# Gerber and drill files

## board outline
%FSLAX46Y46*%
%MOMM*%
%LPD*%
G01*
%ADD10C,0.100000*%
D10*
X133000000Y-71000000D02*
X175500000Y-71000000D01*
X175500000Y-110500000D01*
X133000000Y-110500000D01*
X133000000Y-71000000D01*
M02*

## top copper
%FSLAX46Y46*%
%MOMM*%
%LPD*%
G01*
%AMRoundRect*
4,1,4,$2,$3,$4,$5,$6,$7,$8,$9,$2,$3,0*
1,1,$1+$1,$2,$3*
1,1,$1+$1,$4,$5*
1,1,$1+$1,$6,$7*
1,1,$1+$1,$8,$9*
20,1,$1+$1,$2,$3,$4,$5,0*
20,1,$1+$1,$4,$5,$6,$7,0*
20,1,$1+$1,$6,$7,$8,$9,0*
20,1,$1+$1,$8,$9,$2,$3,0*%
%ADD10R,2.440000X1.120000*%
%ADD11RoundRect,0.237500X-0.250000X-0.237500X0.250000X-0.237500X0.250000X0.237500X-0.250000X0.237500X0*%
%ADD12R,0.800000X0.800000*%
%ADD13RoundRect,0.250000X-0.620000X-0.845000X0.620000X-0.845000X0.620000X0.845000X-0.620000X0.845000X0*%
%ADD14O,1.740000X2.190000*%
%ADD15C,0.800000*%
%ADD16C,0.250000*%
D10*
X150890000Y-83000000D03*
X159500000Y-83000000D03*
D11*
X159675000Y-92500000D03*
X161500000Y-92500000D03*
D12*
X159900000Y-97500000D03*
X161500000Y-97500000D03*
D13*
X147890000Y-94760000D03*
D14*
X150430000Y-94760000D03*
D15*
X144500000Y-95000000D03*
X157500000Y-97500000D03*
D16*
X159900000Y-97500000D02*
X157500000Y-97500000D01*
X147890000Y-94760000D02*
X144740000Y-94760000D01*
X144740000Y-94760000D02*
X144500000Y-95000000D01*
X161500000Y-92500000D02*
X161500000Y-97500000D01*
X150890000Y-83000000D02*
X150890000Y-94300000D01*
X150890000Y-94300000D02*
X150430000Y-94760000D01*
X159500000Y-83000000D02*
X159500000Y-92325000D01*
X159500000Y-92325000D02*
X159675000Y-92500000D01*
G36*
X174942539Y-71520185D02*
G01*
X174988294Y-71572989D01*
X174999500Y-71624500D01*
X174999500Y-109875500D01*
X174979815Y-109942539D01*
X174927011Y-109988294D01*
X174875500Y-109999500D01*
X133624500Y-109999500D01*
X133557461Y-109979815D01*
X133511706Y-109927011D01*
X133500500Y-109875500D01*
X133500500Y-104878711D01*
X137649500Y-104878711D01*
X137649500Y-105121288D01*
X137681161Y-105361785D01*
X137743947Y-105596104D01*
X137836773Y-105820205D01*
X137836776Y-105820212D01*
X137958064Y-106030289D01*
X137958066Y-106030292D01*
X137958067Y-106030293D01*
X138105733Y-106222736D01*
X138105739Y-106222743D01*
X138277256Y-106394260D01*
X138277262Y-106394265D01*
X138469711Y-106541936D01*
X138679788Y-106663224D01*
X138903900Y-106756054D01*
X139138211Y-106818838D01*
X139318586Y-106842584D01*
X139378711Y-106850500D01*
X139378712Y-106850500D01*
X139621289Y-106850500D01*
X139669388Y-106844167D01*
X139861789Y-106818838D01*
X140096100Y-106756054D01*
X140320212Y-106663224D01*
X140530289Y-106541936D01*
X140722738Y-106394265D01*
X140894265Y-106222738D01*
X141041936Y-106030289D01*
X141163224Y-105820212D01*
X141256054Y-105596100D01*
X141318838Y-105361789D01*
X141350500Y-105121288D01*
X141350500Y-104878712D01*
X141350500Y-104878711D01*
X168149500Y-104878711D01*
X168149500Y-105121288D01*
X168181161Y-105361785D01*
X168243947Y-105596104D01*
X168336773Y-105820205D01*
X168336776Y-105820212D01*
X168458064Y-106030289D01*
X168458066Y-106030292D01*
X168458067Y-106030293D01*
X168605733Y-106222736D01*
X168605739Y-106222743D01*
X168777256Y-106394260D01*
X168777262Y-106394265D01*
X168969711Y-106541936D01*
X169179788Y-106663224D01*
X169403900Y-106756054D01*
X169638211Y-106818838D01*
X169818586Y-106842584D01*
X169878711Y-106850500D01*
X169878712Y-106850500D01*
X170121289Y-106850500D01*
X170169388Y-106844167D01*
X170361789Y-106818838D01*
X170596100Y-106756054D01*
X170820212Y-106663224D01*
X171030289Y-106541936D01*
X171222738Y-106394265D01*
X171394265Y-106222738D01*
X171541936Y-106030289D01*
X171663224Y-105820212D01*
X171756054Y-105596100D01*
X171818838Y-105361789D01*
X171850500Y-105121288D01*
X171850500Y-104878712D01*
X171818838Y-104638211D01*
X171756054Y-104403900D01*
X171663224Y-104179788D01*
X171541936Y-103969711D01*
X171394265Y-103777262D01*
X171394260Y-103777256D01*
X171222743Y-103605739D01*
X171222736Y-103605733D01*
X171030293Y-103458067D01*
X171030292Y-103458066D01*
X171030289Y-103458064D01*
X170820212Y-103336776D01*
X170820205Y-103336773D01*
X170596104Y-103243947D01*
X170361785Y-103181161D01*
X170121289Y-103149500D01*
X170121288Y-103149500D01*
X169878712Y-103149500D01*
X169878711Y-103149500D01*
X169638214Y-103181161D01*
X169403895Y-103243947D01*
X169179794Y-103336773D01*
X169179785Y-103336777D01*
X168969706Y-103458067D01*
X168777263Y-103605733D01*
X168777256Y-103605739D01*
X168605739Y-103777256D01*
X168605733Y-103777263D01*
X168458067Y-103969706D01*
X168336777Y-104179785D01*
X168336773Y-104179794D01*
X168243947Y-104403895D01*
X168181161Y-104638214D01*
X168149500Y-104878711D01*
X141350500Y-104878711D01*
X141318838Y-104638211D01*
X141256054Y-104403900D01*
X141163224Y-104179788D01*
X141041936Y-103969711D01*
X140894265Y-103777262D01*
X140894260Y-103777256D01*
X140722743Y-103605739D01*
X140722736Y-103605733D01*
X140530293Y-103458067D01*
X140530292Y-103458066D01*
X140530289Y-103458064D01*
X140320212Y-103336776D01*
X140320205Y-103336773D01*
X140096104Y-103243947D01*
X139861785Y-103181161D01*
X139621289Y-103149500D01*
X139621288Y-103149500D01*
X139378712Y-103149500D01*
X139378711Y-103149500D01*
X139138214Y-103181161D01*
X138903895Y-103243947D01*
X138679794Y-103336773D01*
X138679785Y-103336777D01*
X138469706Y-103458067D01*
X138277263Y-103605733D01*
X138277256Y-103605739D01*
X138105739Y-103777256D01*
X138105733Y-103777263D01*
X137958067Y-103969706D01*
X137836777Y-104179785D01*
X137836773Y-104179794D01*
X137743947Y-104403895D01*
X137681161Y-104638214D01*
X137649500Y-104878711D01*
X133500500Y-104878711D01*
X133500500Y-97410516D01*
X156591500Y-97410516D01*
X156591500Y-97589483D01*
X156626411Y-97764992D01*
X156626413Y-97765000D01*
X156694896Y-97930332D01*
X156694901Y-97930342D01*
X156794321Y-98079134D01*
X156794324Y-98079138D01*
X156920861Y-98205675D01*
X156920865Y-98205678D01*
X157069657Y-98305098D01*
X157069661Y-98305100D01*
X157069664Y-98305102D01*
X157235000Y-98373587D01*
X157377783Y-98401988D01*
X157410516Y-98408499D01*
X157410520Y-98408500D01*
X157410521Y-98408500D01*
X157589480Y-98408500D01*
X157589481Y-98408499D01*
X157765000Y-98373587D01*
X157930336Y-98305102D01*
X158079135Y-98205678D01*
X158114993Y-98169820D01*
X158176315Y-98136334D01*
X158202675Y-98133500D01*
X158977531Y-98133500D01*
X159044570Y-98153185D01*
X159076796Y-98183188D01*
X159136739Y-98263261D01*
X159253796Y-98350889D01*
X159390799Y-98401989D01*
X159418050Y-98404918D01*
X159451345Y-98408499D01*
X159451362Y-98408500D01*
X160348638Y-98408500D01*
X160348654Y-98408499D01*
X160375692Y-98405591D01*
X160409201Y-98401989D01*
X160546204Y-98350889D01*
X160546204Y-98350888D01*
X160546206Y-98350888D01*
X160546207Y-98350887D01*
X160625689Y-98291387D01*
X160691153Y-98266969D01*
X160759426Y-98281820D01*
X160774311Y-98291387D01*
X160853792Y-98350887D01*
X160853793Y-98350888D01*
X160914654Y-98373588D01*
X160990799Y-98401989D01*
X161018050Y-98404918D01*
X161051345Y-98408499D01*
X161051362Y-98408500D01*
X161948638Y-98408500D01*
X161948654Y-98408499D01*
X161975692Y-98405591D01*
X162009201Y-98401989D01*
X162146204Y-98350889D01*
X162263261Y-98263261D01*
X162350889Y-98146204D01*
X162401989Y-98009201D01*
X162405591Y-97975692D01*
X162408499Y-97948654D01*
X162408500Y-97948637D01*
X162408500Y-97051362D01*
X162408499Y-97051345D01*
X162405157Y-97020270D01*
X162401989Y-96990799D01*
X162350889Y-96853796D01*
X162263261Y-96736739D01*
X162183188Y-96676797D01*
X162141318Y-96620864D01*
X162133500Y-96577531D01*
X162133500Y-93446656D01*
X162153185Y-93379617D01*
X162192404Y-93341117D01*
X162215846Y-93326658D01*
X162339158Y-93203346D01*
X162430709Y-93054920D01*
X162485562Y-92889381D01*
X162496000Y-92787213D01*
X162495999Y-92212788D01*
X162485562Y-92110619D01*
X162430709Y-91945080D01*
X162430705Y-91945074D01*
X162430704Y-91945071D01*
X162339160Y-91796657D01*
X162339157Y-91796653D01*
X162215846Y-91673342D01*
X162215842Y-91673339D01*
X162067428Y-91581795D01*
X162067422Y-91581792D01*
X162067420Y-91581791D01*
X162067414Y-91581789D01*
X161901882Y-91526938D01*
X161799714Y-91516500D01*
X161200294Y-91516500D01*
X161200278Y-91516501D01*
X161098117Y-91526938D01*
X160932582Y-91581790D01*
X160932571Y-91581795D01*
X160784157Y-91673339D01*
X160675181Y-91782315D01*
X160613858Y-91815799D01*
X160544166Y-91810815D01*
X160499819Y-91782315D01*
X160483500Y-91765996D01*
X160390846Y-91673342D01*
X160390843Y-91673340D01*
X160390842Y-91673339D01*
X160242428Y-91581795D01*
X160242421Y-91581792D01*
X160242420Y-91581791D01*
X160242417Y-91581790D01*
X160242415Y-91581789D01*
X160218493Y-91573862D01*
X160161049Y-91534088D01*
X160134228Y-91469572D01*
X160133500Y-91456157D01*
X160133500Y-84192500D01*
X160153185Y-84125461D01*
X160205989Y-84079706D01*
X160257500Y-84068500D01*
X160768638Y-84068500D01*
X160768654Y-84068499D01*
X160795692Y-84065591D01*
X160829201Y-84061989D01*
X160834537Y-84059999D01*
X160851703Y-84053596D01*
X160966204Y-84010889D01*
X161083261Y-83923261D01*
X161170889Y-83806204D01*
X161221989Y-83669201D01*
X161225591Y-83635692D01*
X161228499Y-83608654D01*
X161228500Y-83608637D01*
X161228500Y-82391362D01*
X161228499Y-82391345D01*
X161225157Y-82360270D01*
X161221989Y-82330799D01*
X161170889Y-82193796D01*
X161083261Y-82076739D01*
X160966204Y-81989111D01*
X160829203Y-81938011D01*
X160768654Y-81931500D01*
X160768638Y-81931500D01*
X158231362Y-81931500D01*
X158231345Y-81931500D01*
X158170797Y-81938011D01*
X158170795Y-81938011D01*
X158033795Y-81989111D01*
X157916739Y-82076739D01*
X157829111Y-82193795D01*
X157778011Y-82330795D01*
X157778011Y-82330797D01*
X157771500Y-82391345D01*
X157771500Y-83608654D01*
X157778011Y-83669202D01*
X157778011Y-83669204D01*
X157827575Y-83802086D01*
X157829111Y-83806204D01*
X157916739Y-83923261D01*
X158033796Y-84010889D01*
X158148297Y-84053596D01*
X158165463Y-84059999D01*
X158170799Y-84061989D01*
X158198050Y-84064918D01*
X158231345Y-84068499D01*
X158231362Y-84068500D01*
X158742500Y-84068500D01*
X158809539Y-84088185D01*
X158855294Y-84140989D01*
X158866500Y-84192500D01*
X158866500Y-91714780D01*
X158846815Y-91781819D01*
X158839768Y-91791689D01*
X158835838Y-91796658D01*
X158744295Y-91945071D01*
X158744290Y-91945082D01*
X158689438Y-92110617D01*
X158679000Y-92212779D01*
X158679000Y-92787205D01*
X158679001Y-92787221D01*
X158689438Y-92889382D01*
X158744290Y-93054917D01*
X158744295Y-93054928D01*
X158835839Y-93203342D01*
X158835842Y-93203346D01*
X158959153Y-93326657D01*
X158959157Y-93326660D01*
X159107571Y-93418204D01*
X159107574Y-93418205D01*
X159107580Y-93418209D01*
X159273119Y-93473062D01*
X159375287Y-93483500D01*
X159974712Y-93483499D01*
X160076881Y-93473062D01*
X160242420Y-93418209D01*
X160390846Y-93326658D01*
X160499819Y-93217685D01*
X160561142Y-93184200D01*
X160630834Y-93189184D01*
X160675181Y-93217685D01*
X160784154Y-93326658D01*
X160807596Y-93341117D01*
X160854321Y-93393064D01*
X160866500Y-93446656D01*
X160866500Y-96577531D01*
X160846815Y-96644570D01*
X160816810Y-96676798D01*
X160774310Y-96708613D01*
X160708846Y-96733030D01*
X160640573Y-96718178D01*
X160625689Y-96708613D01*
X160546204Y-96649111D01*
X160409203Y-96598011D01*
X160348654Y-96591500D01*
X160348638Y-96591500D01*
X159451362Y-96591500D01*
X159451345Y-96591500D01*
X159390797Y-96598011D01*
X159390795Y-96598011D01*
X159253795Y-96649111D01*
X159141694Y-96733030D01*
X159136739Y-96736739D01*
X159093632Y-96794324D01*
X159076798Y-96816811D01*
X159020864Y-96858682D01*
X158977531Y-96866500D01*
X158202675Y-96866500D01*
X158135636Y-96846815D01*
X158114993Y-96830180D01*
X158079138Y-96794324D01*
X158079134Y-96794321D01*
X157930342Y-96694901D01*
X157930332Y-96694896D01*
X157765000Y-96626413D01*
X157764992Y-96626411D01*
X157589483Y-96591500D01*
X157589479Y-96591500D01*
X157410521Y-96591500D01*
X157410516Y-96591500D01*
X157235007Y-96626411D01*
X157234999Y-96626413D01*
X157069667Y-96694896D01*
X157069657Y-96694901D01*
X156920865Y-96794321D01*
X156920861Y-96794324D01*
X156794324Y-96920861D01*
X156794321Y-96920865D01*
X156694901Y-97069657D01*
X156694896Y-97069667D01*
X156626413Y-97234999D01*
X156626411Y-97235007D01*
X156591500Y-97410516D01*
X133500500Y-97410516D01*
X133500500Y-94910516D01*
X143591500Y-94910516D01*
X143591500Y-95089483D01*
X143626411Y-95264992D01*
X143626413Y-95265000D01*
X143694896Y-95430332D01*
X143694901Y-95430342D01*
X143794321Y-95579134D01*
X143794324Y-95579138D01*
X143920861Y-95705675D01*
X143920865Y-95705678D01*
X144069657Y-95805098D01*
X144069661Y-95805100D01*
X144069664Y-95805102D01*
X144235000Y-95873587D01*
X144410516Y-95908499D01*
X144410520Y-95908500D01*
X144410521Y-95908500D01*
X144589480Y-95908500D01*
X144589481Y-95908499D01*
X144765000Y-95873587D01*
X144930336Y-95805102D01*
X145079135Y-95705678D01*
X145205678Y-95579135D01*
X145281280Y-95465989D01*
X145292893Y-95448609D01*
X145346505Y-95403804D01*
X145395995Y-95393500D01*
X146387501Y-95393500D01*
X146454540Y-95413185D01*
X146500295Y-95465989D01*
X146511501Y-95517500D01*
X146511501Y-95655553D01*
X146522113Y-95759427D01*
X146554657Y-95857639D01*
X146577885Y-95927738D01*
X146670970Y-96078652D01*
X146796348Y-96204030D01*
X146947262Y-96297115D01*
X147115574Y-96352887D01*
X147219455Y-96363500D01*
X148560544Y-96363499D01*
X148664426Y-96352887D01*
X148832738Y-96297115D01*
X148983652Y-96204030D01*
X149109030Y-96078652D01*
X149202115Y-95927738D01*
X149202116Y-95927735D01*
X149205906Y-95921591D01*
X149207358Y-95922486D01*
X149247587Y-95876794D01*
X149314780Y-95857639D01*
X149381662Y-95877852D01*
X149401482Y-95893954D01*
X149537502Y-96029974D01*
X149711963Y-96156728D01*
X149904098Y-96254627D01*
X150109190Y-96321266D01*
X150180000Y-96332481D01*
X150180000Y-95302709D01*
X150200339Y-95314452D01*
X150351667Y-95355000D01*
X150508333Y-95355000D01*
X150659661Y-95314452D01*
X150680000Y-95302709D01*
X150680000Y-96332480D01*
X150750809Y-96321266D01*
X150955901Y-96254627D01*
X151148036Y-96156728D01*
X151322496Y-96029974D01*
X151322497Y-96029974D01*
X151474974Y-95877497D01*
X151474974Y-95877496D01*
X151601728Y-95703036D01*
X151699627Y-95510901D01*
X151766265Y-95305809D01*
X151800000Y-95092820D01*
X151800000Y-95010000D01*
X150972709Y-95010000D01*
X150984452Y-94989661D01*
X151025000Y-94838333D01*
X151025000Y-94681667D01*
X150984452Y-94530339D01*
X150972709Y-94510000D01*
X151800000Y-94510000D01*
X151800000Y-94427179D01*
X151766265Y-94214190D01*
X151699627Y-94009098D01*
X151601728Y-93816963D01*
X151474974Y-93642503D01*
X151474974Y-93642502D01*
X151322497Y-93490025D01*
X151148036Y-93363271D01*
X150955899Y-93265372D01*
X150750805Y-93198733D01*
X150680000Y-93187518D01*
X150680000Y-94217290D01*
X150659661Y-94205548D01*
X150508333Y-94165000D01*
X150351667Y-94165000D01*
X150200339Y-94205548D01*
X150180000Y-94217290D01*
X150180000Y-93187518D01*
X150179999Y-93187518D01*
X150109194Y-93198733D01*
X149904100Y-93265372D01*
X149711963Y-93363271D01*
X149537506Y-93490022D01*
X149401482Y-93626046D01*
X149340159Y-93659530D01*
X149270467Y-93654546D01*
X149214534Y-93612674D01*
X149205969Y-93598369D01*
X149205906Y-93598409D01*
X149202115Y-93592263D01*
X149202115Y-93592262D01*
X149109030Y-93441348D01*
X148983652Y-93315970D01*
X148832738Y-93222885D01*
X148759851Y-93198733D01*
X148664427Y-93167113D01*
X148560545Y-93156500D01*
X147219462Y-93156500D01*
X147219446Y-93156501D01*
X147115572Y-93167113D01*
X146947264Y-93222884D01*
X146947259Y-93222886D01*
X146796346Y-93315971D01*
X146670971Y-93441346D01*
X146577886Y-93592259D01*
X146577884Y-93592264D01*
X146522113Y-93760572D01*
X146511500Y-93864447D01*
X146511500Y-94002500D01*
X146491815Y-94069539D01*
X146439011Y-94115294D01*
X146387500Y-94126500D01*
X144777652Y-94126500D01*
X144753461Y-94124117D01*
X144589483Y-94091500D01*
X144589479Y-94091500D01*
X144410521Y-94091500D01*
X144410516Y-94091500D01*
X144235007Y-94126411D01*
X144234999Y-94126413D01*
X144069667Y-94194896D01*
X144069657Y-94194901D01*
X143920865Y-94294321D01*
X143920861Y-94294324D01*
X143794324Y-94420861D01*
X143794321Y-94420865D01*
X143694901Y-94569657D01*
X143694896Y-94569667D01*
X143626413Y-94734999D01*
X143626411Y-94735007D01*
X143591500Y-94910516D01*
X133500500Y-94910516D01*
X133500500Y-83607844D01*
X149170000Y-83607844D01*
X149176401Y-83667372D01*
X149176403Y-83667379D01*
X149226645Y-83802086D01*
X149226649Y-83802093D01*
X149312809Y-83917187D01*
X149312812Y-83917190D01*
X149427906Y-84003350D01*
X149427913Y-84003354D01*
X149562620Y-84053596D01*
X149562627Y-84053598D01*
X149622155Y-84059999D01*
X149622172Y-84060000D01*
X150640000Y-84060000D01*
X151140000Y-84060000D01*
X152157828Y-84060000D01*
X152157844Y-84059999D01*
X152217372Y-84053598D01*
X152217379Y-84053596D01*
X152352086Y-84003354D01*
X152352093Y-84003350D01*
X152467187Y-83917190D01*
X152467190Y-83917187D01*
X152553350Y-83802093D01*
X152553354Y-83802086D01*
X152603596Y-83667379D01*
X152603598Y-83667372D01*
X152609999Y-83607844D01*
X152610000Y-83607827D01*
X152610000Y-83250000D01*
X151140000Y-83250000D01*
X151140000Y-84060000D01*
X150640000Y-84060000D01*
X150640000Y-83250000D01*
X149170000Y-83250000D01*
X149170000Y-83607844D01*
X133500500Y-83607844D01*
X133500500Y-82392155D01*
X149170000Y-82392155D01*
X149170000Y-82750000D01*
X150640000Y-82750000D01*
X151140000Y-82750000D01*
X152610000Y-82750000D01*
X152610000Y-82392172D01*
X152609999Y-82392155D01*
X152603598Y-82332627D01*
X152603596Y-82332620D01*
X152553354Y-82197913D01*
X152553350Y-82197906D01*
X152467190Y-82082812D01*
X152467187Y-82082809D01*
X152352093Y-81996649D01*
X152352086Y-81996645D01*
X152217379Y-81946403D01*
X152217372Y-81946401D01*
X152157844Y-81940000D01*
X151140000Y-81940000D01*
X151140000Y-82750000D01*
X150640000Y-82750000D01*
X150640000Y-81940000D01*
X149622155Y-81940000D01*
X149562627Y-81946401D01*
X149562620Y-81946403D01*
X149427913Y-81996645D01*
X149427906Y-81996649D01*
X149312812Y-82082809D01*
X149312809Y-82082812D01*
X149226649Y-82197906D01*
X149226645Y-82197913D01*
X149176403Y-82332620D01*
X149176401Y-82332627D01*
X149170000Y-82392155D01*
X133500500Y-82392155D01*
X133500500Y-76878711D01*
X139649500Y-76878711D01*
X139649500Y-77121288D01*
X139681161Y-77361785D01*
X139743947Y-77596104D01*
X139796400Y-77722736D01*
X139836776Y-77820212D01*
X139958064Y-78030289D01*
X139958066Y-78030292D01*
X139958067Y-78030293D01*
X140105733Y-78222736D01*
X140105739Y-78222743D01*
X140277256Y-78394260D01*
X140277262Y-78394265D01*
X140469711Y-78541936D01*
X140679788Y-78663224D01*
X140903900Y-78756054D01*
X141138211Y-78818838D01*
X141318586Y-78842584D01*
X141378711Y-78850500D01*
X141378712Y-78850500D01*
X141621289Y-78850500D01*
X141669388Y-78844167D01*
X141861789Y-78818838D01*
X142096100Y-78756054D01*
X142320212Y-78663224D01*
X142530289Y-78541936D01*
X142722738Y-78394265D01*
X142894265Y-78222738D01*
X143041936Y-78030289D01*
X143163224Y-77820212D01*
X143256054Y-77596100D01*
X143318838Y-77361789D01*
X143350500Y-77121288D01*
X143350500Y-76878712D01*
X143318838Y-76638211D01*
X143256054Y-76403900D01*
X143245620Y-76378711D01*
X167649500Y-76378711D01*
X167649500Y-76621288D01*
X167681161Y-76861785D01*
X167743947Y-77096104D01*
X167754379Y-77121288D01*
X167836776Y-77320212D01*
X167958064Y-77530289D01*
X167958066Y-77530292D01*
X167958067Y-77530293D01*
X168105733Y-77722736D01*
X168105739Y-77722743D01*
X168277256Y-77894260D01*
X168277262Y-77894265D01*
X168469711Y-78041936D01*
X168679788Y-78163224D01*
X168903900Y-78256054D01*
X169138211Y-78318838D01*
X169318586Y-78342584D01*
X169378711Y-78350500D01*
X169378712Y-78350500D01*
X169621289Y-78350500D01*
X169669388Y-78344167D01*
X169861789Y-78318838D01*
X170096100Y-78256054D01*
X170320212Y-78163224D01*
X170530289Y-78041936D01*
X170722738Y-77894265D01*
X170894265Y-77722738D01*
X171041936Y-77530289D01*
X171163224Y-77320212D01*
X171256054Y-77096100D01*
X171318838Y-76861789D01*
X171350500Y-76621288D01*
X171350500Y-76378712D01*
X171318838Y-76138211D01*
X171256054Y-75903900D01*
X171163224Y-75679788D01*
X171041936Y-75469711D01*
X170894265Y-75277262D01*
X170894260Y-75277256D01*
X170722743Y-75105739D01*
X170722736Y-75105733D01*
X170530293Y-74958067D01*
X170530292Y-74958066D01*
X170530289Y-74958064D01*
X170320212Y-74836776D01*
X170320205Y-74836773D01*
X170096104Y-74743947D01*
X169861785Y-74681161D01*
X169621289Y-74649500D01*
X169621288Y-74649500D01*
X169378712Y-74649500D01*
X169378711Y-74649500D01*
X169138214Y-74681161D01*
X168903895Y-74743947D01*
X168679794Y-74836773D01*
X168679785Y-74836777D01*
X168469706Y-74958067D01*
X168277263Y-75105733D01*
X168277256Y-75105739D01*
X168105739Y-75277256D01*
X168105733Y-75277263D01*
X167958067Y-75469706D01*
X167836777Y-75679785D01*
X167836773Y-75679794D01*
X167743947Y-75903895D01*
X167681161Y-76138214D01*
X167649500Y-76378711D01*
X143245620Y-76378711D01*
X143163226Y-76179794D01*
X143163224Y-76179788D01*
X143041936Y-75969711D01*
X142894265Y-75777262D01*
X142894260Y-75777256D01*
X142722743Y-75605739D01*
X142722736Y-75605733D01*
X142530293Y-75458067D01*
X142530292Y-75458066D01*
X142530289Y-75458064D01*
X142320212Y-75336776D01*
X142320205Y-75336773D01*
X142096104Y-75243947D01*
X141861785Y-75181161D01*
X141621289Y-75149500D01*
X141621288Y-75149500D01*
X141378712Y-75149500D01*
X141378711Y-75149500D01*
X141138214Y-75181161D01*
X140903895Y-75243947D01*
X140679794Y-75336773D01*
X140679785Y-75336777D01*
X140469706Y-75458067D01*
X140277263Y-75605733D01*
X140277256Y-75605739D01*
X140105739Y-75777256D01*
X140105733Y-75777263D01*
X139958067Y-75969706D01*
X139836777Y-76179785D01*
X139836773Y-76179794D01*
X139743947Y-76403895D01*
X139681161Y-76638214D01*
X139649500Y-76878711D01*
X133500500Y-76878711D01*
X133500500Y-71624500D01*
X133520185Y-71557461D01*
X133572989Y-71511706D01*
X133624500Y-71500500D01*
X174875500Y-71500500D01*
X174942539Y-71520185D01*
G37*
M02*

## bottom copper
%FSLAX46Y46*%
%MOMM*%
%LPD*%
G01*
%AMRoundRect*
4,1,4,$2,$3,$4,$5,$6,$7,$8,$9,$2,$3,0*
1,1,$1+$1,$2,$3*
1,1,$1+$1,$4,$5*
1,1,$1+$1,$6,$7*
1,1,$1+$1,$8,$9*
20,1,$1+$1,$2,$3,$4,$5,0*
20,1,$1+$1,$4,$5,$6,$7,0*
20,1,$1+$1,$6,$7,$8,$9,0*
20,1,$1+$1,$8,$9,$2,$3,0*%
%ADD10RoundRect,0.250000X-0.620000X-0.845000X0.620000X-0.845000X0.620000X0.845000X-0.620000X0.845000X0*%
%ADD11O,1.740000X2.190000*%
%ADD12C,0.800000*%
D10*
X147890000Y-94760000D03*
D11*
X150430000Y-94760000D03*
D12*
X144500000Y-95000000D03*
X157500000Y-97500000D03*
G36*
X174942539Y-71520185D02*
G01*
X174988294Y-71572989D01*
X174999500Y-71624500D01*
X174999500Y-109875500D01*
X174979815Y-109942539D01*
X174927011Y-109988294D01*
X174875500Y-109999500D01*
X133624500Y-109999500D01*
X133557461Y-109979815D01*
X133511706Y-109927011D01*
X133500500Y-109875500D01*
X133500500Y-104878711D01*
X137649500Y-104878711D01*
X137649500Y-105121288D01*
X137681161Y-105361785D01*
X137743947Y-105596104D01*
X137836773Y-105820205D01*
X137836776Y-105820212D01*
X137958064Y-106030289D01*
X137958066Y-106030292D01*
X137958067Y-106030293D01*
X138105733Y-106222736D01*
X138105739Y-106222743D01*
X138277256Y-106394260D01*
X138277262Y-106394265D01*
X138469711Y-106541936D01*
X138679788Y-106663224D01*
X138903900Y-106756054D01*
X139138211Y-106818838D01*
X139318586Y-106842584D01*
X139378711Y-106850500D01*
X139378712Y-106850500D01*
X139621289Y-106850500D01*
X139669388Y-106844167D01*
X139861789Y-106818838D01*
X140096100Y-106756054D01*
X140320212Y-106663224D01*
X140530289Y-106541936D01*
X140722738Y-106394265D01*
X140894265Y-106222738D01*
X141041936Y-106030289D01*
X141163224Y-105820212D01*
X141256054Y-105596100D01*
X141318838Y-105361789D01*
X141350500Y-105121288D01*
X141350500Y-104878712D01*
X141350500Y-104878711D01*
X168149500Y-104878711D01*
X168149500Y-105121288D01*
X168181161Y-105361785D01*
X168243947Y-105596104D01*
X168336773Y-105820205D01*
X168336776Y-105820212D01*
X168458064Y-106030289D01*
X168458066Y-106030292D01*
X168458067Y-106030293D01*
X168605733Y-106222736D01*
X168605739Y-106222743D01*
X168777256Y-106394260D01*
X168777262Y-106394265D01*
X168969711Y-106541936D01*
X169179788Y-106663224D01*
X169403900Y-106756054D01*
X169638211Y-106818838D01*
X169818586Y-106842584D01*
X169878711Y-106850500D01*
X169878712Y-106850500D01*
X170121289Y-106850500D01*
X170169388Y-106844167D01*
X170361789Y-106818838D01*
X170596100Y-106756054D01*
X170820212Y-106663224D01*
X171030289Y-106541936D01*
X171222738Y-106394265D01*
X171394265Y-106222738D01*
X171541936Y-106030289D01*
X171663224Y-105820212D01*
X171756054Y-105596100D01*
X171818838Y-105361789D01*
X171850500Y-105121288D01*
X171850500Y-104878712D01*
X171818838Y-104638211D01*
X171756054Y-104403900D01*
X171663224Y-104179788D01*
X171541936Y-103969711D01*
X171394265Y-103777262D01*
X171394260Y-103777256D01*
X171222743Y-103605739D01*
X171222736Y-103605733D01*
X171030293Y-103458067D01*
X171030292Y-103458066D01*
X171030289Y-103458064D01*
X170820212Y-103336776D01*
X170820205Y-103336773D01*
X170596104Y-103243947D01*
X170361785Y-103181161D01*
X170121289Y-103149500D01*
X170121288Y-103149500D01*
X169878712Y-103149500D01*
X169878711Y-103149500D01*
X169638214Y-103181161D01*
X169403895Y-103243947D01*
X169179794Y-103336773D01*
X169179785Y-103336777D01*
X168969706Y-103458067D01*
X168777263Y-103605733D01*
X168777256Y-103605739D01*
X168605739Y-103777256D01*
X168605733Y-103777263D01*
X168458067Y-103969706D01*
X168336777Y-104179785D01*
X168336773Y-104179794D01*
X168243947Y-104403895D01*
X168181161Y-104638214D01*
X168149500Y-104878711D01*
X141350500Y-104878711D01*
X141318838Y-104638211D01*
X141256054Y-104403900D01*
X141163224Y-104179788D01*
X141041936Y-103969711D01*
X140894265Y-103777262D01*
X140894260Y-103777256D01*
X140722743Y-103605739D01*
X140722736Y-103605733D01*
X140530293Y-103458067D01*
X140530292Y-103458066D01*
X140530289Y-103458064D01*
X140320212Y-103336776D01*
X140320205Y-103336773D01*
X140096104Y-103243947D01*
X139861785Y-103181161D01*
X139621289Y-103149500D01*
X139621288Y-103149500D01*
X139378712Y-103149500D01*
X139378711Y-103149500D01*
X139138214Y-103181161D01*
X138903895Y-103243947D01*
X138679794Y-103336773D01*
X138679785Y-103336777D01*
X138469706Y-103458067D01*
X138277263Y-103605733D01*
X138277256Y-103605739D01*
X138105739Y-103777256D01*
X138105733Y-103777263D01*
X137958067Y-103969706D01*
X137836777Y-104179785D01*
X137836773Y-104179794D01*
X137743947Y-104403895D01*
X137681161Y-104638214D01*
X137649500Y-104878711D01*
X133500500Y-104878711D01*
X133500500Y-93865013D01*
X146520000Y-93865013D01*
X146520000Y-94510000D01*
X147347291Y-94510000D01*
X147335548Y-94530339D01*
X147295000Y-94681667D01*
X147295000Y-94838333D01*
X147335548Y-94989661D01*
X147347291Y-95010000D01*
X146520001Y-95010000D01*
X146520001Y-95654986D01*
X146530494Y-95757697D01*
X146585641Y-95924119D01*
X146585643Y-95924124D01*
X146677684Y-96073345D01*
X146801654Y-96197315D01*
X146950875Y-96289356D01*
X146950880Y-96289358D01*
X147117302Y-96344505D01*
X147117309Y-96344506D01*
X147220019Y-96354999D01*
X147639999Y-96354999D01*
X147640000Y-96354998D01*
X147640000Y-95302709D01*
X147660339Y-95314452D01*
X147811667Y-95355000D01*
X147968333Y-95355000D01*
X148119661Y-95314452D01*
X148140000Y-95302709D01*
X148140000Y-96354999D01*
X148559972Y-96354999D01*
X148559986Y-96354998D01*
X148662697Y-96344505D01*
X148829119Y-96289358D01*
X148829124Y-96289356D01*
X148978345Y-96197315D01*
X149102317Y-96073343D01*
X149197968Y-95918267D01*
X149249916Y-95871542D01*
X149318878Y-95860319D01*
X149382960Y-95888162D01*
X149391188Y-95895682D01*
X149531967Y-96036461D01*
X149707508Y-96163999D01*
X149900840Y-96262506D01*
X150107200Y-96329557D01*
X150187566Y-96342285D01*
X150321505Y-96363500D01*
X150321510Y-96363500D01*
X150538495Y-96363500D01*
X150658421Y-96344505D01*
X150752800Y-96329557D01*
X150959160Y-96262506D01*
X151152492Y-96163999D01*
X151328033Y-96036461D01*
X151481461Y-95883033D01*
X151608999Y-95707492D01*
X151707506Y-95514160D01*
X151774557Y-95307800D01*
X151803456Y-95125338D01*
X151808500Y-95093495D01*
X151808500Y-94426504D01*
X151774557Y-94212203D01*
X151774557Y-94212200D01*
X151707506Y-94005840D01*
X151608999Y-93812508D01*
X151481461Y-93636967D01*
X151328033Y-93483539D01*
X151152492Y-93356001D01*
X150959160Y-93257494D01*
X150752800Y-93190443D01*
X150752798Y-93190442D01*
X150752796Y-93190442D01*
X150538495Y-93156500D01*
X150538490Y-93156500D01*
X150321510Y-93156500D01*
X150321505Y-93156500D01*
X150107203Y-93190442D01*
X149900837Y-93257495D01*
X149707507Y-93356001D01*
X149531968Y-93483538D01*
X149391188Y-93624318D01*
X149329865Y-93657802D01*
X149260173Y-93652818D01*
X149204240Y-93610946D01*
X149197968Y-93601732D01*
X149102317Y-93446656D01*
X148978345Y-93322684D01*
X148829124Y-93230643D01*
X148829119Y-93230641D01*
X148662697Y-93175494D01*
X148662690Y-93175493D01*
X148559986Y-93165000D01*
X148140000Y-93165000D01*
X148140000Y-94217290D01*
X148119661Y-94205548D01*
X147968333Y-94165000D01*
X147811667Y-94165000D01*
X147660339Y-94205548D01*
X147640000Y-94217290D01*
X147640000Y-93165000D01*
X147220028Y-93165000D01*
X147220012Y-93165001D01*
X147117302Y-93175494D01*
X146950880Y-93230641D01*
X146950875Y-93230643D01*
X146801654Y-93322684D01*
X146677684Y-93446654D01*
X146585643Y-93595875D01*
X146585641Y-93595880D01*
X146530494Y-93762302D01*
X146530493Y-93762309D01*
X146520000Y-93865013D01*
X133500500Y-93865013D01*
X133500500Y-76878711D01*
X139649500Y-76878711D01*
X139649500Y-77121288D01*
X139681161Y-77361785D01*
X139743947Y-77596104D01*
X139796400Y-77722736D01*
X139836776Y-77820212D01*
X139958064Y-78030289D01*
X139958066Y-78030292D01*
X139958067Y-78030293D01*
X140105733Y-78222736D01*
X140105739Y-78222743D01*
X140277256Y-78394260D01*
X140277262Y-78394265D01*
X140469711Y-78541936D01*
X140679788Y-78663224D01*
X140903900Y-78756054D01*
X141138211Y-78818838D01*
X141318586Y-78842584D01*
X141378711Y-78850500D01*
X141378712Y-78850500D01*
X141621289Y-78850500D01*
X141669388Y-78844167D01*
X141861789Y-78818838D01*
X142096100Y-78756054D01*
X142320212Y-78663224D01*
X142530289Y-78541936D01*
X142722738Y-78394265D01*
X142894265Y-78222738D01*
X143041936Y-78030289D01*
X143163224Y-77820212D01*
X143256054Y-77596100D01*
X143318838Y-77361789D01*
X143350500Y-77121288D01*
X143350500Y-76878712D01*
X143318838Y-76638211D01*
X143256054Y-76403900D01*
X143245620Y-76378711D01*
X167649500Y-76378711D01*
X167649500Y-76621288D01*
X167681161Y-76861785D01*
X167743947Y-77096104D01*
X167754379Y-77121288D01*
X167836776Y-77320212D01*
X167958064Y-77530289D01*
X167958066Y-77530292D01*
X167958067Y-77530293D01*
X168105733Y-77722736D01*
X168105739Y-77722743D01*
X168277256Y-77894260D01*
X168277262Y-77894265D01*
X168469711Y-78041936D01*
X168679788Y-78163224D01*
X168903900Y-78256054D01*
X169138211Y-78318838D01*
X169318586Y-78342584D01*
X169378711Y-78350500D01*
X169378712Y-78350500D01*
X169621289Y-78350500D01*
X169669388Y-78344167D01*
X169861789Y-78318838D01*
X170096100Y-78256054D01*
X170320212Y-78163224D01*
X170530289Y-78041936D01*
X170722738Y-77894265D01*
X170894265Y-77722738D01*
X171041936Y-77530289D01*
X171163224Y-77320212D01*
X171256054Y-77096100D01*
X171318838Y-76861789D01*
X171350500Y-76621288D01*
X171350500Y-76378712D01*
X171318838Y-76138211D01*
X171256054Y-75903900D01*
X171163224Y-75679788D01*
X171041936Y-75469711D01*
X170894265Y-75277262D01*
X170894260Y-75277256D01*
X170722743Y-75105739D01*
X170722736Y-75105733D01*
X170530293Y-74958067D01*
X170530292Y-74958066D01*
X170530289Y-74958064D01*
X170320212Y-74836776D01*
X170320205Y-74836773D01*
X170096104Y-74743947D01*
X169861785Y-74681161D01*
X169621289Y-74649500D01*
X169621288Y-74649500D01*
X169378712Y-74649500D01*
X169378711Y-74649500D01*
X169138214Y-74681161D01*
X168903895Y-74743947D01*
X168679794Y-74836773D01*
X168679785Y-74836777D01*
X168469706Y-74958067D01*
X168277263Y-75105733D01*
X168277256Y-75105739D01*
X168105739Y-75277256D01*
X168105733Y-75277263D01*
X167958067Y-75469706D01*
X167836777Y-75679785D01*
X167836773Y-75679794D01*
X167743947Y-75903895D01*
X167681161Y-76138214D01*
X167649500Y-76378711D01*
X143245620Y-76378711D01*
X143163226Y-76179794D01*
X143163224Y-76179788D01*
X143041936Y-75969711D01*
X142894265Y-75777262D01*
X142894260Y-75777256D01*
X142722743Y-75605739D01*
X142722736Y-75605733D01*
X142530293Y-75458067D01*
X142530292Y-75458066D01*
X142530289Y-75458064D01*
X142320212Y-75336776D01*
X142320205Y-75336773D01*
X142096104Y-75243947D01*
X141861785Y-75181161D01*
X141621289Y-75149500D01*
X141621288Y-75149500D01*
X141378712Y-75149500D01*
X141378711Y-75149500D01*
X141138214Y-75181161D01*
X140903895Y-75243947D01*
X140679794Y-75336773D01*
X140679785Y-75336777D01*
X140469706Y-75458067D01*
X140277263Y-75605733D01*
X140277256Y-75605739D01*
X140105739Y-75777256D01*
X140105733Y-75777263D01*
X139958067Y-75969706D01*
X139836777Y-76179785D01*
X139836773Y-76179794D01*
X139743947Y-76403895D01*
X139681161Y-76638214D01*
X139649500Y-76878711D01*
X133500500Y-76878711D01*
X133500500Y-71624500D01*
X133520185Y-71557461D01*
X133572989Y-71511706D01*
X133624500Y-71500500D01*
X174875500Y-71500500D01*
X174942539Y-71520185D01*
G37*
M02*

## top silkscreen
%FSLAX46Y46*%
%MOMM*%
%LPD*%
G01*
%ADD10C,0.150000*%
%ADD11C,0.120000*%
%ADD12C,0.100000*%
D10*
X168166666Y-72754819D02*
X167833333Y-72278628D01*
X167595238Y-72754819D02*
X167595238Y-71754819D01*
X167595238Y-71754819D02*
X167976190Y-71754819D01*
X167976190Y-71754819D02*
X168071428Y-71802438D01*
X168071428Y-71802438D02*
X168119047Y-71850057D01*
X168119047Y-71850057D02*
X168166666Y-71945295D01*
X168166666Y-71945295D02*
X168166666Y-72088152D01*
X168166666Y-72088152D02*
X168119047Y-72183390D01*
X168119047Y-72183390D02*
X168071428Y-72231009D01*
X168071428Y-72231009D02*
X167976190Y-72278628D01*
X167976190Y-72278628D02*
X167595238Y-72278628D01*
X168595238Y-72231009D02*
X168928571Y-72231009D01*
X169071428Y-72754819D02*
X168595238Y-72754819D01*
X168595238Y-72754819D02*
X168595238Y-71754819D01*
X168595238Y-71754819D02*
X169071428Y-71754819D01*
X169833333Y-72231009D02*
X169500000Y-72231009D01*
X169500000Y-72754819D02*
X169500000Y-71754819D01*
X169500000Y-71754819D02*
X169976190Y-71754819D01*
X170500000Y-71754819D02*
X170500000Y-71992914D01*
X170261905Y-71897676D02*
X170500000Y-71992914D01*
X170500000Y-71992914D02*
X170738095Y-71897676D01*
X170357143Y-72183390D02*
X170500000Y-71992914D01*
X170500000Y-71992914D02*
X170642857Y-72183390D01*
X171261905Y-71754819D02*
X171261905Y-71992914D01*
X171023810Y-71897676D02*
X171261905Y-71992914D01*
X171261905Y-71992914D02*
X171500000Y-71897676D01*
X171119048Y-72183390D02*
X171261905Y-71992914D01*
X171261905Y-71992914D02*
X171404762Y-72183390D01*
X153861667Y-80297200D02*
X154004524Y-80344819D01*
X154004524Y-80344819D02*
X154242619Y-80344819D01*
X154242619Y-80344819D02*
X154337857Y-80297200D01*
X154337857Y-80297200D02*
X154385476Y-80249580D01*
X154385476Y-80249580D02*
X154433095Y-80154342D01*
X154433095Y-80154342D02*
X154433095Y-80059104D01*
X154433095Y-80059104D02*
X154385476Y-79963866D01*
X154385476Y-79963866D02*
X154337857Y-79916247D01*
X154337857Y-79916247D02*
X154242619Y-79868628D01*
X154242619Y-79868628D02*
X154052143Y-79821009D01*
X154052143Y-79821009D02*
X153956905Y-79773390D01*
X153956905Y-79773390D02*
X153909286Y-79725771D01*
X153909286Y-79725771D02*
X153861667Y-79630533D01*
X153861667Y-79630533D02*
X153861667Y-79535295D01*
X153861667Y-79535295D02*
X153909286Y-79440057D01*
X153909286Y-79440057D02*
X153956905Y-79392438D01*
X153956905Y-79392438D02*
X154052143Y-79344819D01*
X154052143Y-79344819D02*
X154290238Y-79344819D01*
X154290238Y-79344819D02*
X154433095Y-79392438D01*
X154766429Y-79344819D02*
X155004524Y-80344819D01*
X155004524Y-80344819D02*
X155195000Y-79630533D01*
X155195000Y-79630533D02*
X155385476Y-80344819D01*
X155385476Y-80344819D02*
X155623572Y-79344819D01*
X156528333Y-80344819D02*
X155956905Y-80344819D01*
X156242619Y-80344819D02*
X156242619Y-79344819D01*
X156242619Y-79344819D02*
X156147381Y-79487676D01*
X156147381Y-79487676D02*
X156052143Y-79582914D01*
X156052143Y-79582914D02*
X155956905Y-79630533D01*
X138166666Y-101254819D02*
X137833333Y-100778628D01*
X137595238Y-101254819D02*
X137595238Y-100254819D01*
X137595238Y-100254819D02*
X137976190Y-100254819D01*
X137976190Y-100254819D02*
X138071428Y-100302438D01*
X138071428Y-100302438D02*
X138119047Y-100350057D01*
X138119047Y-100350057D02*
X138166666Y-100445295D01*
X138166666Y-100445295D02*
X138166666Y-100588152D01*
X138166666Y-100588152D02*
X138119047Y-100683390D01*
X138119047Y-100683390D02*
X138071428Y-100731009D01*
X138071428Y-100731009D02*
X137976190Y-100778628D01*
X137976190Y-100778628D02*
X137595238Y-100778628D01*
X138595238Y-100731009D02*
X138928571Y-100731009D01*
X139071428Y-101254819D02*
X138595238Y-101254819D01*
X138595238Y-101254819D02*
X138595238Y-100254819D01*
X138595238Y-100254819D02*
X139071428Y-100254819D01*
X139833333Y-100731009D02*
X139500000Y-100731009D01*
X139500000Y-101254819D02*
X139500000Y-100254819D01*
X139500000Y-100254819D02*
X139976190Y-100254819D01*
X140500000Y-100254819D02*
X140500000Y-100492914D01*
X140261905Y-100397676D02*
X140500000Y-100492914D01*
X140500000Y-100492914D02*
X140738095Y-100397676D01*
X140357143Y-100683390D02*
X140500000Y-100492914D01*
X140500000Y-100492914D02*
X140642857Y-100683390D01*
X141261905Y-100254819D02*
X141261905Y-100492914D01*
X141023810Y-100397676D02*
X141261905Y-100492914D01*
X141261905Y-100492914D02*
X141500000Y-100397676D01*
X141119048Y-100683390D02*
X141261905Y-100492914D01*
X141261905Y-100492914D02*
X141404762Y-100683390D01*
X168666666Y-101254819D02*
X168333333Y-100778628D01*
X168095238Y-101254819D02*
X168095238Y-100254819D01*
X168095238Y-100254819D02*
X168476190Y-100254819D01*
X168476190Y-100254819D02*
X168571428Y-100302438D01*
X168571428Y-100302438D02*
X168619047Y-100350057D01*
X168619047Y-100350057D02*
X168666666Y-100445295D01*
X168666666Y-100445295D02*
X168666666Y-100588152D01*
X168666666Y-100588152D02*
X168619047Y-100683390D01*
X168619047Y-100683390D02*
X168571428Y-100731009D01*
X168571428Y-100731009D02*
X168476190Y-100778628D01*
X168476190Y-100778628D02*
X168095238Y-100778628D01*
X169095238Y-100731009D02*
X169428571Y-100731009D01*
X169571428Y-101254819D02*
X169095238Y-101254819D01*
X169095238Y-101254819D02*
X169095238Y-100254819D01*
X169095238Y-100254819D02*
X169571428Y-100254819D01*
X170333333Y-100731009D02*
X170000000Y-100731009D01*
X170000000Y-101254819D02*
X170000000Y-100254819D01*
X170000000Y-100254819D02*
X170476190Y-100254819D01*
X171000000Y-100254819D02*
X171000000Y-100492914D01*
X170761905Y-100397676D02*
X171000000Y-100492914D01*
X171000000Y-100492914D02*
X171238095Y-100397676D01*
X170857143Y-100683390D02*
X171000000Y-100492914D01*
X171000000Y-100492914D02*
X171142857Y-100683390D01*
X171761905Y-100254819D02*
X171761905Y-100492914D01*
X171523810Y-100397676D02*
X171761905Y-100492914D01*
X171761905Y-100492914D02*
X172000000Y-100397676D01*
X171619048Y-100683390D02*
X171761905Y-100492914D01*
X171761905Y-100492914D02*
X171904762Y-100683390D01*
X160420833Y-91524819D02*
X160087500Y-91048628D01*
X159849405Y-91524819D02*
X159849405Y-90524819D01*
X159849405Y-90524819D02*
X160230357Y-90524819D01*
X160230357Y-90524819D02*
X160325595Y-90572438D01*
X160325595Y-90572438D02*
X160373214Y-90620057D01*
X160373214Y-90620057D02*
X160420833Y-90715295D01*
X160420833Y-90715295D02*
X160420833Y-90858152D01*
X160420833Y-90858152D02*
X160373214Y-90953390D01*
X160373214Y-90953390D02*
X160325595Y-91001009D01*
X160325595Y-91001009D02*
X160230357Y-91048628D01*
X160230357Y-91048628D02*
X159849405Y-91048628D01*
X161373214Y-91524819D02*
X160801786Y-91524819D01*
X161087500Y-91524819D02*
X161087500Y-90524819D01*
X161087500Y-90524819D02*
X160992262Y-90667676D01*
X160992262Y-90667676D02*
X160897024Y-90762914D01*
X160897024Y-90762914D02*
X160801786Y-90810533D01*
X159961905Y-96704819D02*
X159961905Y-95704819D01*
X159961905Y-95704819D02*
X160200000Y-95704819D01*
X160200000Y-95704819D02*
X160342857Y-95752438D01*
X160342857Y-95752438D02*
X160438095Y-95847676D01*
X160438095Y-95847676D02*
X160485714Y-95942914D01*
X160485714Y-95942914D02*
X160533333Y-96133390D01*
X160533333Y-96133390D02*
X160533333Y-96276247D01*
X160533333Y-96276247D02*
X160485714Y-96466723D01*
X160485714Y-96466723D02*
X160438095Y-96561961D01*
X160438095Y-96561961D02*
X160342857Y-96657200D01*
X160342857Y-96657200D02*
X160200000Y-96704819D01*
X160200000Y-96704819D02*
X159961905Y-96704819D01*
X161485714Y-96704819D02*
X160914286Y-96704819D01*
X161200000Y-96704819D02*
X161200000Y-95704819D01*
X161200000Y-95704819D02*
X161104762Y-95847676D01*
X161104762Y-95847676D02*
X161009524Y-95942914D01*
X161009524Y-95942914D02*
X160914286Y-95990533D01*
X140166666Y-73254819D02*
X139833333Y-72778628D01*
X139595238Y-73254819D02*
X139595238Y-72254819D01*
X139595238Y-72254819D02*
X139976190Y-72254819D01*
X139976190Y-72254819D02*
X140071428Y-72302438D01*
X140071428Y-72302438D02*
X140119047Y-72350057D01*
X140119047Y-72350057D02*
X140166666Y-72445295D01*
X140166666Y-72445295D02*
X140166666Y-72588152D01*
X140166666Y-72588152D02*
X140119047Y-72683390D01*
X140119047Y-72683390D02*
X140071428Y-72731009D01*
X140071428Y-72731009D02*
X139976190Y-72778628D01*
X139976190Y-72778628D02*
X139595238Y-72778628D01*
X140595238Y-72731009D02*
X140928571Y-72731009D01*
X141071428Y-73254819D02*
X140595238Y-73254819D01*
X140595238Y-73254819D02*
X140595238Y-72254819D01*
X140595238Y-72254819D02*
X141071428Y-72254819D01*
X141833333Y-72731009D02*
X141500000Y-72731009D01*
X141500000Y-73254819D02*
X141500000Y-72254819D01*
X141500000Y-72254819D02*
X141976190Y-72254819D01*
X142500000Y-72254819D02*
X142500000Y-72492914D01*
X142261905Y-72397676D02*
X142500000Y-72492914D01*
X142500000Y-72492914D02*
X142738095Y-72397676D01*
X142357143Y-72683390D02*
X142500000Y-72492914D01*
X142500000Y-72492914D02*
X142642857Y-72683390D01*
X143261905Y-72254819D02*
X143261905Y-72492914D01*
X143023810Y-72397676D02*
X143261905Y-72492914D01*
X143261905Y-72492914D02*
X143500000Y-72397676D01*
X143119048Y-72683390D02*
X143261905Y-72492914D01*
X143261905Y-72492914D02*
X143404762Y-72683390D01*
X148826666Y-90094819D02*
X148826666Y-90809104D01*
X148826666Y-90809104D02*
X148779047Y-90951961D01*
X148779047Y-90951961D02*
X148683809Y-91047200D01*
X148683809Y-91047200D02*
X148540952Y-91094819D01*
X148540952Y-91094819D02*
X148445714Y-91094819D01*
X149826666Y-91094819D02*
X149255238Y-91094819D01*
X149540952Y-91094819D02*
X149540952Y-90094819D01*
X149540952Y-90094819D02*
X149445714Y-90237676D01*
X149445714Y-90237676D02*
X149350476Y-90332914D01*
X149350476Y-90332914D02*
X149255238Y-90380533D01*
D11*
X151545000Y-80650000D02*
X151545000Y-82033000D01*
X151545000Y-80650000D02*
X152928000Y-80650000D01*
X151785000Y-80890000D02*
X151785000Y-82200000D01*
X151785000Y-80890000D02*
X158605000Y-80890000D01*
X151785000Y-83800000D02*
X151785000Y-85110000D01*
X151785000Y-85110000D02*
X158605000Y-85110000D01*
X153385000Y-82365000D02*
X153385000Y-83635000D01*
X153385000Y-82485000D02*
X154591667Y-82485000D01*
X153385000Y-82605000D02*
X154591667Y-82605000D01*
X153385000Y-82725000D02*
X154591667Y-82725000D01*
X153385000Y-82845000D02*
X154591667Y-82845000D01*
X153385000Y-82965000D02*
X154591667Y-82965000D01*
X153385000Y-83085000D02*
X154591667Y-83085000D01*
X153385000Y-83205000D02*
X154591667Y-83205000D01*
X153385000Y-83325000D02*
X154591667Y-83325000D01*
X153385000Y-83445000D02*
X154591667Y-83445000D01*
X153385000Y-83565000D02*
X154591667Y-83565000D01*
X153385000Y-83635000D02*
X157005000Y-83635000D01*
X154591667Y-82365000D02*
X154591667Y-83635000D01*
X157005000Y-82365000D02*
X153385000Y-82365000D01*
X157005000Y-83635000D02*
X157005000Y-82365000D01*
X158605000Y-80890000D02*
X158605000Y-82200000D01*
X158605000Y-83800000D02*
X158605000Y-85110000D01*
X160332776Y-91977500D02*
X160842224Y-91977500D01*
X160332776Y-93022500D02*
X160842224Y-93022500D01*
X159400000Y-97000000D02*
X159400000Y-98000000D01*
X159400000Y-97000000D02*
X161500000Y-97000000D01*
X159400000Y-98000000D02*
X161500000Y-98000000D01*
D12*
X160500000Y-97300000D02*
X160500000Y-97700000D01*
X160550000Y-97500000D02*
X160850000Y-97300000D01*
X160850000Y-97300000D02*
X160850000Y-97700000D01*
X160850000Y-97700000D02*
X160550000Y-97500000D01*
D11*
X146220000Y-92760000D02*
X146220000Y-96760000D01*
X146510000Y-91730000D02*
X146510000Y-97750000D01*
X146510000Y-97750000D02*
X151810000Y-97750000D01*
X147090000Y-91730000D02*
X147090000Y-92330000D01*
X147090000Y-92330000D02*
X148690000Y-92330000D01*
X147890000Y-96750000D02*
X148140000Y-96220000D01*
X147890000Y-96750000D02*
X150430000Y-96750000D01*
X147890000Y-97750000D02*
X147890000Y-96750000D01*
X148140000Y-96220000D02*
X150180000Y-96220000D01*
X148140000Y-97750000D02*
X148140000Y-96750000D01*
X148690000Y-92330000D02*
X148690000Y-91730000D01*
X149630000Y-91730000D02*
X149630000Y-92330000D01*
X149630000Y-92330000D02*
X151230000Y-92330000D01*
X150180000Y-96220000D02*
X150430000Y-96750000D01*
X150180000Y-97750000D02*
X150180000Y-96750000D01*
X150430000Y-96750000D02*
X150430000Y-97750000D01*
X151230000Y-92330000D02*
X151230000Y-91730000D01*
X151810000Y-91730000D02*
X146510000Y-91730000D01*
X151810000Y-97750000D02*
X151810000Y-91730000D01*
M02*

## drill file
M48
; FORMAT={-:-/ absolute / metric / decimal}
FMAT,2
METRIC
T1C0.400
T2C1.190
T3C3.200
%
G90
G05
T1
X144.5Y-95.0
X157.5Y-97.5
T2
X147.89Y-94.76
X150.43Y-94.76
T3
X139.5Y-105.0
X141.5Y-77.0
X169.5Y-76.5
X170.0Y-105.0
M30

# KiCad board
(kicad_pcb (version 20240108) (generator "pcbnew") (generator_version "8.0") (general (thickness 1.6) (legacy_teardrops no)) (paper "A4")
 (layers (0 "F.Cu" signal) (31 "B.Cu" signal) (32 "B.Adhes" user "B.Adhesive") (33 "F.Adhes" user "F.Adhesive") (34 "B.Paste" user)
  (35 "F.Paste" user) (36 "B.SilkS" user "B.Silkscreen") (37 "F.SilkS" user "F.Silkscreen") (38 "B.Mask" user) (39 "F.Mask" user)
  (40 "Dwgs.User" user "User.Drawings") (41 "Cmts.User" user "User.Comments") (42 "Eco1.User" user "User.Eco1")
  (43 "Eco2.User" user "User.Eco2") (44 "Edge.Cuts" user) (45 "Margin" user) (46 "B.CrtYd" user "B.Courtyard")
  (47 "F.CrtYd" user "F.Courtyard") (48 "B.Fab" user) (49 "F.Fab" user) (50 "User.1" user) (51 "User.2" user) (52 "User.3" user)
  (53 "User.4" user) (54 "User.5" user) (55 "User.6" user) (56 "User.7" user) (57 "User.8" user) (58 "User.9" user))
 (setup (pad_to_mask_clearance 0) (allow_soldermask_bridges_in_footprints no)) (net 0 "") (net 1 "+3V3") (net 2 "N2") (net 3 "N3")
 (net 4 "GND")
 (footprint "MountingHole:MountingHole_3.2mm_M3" (layer "F.Cu") (at 169.5 76.5)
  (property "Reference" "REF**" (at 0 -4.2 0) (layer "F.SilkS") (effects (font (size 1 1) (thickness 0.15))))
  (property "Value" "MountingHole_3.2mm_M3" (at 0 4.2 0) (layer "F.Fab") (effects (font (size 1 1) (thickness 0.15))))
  (pad "" np_thru_hole circle (at 0 0) (size 3.2 3.2) (drill 3.2) (layers "*.Cu" "*.Mask")))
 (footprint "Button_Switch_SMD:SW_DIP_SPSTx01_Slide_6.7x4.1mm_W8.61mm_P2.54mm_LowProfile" (layer "F.Cu") (at 155.195 83)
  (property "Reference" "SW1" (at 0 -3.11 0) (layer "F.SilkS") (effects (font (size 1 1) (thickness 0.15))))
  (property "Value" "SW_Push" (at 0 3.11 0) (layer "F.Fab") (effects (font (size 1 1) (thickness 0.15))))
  (fp_line (start -3.65 -2.35) (end -3.65 -0.967) (stroke (width 0.12) (type solid)) (layer "F.SilkS"))
  (fp_line (start -3.65 -2.35) (end -2.267 -2.35) (stroke (width 0.12) (type solid)) (layer "F.SilkS"))
  (fp_line (start -3.41 -2.11) (end -3.41 -0.8) (stroke (width 0.12) (type solid)) (layer "F.SilkS"))
  (fp_line (start -3.41 -2.11) (end 3.41 -2.11) (stroke (width 0.12) (type solid)) (layer "F.SilkS"))
  (fp_line (start -3.41 0.8) (end -3.41 2.11) (stroke (width 0.12) (type solid)) (layer "F.SilkS"))
  (fp_line (start -3.41 2.11) (end 3.41 2.11) (stroke (width 0.12) (type solid)) (layer "F.SilkS"))
  (fp_line (start -1.81 -0.635) (end -1.81 0.635) (stroke (width 0.12) (type solid)) (layer "F.SilkS"))
  (fp_line (start -1.81 -0.515) (end -0.603333 -0.515) (stroke (width 0.12) (type solid)) (layer "F.SilkS"))
  (fp_line (start -1.81 -0.395) (end -0.603333 -0.395) (stroke (width 0.12) (type solid)) (layer "F.SilkS"))
  (fp_line (start -1.81 -0.275) (end -0.603333 -0.275) (stroke (width 0.12) (type solid)) (layer "F.SilkS"))
  (fp_line (start -1.81 -0.155) (end -0.603333 -0.155) (stroke (width 0.12) (type solid)) (layer "F.SilkS"))
  (fp_line (start -1.81 -0.035) (end -0.603333 -0.035) (stroke (width 0.12) (type solid)) (layer "F.SilkS"))
  (fp_line (start -1.81 0.085) (end -0.603333 0.085) (stroke (width 0.12) (type solid)) (layer "F.SilkS"))
  (fp_line (start -1.81 0.205) (end -0.603333 0.205) (stroke (width 0.12) (type solid)) (layer "F.SilkS"))
  (fp_line (start -1.81 0.325) (end -0.603333 0.325) (stroke (width 0.12) (type solid)) (layer "F.SilkS"))
  (fp_line (start -1.81 0.445) (end -0.603333 0.445) (stroke (width 0.12) (type solid)) (layer "F.SilkS"))
  (fp_line (start -1.81 0.565) (end -0.603333 0.565) (stroke (width 0.12) (type solid)) (layer "F.SilkS"))
  (fp_line (start -1.81 0.635) (end 1.81 0.635) (stroke (width 0.12) (type solid)) (layer "F.SilkS"))
  (fp_line (start -0.603333 -0.635) (end -0.603333 0.635) (stroke (width 0.12) (type solid)) (layer "F.SilkS"))
  (fp_line (start 1.81 -0.635) (end -1.81 -0.635) (stroke (width 0.12) (type solid)) (layer "F.SilkS"))
  (fp_line (start 1.81 0.635) (end 1.81 -0.635) (stroke (width 0.12) (type solid)) (layer "F.SilkS"))
  (fp_line (start 3.41 -2.11) (end 3.41 -0.8) (stroke (width 0.12) (type solid)) (layer "F.SilkS"))
  (fp_line (start 3.41 0.8) (end 3.41 2.11) (stroke (width 0.12) (type solid)) (layer "F.SilkS"))
  (pad "1" smd rect (at -4.305 0) (size 2.44 1.12) (layers "F.Cu" "F.Paste" "F.Mask") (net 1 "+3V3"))
  (pad "2" smd rect (at 4.305 0) (size 2.44 1.12) (layers "F.Cu" "F.Paste" "F.Mask") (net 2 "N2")))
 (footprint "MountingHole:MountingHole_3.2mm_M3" (layer "F.Cu") (at 139.5 105)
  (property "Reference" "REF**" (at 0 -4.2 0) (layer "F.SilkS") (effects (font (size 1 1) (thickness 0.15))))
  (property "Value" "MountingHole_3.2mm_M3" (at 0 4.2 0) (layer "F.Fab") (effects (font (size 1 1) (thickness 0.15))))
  (pad "" np_thru_hole circle (at 0 0) (size 3.2 3.2) (drill 3.2) (layers "*.Cu" "*.Mask")))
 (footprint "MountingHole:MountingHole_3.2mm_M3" (layer "F.Cu") (at 170 105)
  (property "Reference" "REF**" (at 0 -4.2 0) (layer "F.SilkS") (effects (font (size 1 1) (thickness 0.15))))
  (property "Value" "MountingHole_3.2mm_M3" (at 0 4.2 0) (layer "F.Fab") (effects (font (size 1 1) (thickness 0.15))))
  (pad "" np_thru_hole circle (at 0 0) (size 3.2 3.2) (drill 3.2) (layers "*.Cu" "*.Mask")))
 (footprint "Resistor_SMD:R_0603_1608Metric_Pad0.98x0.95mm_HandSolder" (layer "F.Cu") (at 160.5875 92.5)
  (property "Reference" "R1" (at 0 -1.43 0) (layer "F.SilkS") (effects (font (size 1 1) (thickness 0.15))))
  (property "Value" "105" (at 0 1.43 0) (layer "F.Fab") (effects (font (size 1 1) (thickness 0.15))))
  (fp_line (start -0.254724 -0.5225) (end 0.254724 -0.5225) (stroke (width 0.12) (type solid)) (layer "F.SilkS"))
  (fp_line (start -0.254724 0.5225) (end 0.254724 0.5225) (stroke (width 0.12) (type solid)) (layer "F.SilkS"))
  (pad "1" smd roundrect (at -0.9125 0) (size 0.975 0.95) (layers "F.Cu" "F.Paste" "F.Mask") (roundrect_rratio 0.25) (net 2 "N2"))
  (pad "2" smd roundrect (at 0.9125 0) (size 0.975 0.95) (layers "F.Cu" "F.Paste" "F.Mask") (roundrect_rratio 0.25) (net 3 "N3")))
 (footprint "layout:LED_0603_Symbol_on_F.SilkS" (layer "F.Cu") (at 160.7 97.5)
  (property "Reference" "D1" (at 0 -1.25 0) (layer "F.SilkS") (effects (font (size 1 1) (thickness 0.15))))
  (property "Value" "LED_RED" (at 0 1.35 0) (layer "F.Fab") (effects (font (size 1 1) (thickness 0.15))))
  (fp_line (start -1.3 -0.5) (end -1.3 0.5) (stroke (width 0.12) (type solid)) (layer "F.SilkS"))
  (fp_line (start -1.3 -0.5) (end 0.8 -0.5) (stroke (width 0.12) (type solid)) (layer "F.SilkS"))
  (fp_line (start -1.3 0.5) (end 0.8 0.5) (stroke (width 0.12) (type solid)) (layer "F.SilkS"))
  (fp_line (start -0.2 -0.2) (end -0.2 0.2) (stroke (width 0.1) (type solid)) (layer "F.SilkS"))
  (fp_line (start -0.15 0) (end 0.15 -0.2) (stroke (width 0.1) (type solid)) (layer "F.SilkS"))
  (fp_line (start 0.15 -0.2) (end 0.15 0.2) (stroke (width 0.1) (type solid)) (layer "F.SilkS"))
  (fp_line (start 0.15 0.2) (end -0.15 0) (stroke (width 0.1) (type solid)) (layer "F.SilkS"))
  (pad "1" smd rect (at -0.8 0 180) (size 0.8 0.8) (layers "F.Cu" "F.Paste" "F.Mask") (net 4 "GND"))
  (pad "2" smd rect (at 0.8 0 180) (size 0.8 0.8) (layers "F.Cu" "F.Paste" "F.Mask") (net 3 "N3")))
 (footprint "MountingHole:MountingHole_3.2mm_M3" (layer "F.Cu") (at 141.5 77)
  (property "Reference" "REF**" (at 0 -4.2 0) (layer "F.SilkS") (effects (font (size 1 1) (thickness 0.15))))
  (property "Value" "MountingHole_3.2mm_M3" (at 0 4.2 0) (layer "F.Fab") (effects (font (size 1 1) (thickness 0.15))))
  (pad "" np_thru_hole circle (at 0 0) (size 3.2 3.2) (drill 3.2) (layers "*.Cu" "*.Mask")))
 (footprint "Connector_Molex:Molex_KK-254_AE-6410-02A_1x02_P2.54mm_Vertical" (layer "F.Cu") (at 147.89 94.76)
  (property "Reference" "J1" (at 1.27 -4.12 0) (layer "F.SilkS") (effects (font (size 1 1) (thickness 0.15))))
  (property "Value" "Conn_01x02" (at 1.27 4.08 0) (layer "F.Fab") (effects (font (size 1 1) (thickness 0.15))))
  (fp_line (start -1.67 -2) (end -1.67 2) (stroke (width 0.12) (type solid)) (layer "F.SilkS"))
  (fp_line (start -1.38 -3.03) (end -1.38 2.99) (stroke (width 0.12) (type solid)) (layer "F.SilkS"))
  (fp_line (start -1.38 2.99) (end 3.92 2.99) (stroke (width 0.12) (type solid)) (layer "F.SilkS"))
  (fp_line (start -0.8 -3.03) (end -0.8 -2.43) (stroke (width 0.12) (type solid)) (layer "F.SilkS"))
  (fp_line (start -0.8 -2.43) (end 0.8 -2.43) (stroke (width 0.12) (type solid)) (layer "F.SilkS"))
  (fp_line (start 0 1.99) (end 0.25 1.46) (stroke (width 0.12) (type solid)) (layer "F.SilkS"))
  (fp_line (start 0 1.99) (end 2.54 1.99) (stroke (width 0.12) (type solid)) (layer "F.SilkS"))
  (fp_line (start 0 2.99) (end 0 1.99) (stroke (width 0.12) (type solid)) (layer "F.SilkS"))
  (fp_line (start 0.25 1.46) (end 2.29 1.46) (stroke (width 0.12) (type solid)) (layer "F.SilkS"))
  (fp_line (start 0.25 2.99) (end 0.25 1.99) (stroke (width 0.12) (type solid)) (layer "F.SilkS"))
  (fp_line (start 0.8 -2.43) (end 0.8 -3.03) (stroke (width 0.12) (type solid)) (layer "F.SilkS"))
  (fp_line (start 1.74 -3.03) (end 1.74 -2.43) (stroke (width 0.12) (type solid)) (layer "F.SilkS"))
  (fp_line (start 1.74 -2.43) (end 3.34 -2.43) (stroke (width 0.12) (type solid)) (layer "F.SilkS"))
  (fp_line (start 2.29 1.46) (end 2.54 1.99) (stroke (width 0.12) (type solid)) (layer "F.SilkS"))
  (fp_line (start 2.29 2.99) (end 2.29 1.99) (stroke (width 0.12) (type solid)) (layer "F.SilkS"))
  (fp_line (start 2.54 1.99) (end 2.54 2.99) (stroke (width 0.12) (type solid)) (layer "F.SilkS"))
  (fp_line (start 3.34 -2.43) (end 3.34 -3.03) (stroke (width 0.12) (type solid)) (layer "F.SilkS"))
  (fp_line (start 3.92 -3.03) (end -1.38 -3.03) (stroke (width 0.12) (type solid)) (layer "F.SilkS"))
  (fp_line (start 3.92 2.99) (end 3.92 -3.03) (stroke (width 0.12) (type solid)) (layer "F.SilkS"))
  (pad "1" thru_hole roundrect (at 0 0) (size 1.74 2.19) (drill 1.19) (layers "*.Cu" "*.Mask") (remove_unused_layers no)
   (roundrect_rratio 0.143678) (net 4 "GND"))
  (pad "2" thru_hole oval (at 2.54 0) (size 1.74 2.19) (drill 1.19) (layers "*.Cu" "*.Mask") (remove_unused_layers no) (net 1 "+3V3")))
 (gr_rect (start 133 71) (end 175.5 110.5) (stroke (width 0.1) (type default)) (fill none) (layer "Edge.Cuts"))
 (segment (start 159.9 97.5) (end 157.5 97.5) (width 0.25) (layer "F.Cu") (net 4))
 (segment (start 147.89 94.76) (end 144.74 94.76) (width 0.25) (layer "F.Cu") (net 4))
 (segment (start 144.74 94.76) (end 144.5 95) (width 0.25) (layer "F.Cu") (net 4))
 (via (at 144.5 95) (size 0.8) (drill 0.4) (layers "F.Cu" "B.Cu") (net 4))
 (via (at 157.5 97.5) (size 0.8) (drill 0.4) (layers "F.Cu" "B.Cu") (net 4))
 (segment (start 161.5 92.5) (end 161.5 97.5) (width 0.25) (layer "F.Cu") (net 3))
 (segment (start 150.89 83) (end 150.89 94.3) (width 0.25) (layer "F.Cu") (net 1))
 (segment (start 150.89 94.3) (end 150.43 94.76) (width 0.25) (layer "F.Cu") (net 1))
 (segment (start 159.5 83) (end 159.5 92.325) (width 0.25) (layer "F.Cu") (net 2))
 (segment (start 159.5 92.325) (end 159.675 92.5) (width 0.25) (layer "F.Cu") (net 2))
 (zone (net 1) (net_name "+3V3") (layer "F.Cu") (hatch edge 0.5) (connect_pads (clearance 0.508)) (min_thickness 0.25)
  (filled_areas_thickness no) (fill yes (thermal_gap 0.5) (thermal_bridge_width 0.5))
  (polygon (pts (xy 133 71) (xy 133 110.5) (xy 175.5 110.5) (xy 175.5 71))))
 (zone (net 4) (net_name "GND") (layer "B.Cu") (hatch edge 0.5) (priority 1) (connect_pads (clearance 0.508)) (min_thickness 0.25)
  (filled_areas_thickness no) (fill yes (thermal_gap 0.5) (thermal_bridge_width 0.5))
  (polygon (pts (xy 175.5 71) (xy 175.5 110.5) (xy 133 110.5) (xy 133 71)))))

